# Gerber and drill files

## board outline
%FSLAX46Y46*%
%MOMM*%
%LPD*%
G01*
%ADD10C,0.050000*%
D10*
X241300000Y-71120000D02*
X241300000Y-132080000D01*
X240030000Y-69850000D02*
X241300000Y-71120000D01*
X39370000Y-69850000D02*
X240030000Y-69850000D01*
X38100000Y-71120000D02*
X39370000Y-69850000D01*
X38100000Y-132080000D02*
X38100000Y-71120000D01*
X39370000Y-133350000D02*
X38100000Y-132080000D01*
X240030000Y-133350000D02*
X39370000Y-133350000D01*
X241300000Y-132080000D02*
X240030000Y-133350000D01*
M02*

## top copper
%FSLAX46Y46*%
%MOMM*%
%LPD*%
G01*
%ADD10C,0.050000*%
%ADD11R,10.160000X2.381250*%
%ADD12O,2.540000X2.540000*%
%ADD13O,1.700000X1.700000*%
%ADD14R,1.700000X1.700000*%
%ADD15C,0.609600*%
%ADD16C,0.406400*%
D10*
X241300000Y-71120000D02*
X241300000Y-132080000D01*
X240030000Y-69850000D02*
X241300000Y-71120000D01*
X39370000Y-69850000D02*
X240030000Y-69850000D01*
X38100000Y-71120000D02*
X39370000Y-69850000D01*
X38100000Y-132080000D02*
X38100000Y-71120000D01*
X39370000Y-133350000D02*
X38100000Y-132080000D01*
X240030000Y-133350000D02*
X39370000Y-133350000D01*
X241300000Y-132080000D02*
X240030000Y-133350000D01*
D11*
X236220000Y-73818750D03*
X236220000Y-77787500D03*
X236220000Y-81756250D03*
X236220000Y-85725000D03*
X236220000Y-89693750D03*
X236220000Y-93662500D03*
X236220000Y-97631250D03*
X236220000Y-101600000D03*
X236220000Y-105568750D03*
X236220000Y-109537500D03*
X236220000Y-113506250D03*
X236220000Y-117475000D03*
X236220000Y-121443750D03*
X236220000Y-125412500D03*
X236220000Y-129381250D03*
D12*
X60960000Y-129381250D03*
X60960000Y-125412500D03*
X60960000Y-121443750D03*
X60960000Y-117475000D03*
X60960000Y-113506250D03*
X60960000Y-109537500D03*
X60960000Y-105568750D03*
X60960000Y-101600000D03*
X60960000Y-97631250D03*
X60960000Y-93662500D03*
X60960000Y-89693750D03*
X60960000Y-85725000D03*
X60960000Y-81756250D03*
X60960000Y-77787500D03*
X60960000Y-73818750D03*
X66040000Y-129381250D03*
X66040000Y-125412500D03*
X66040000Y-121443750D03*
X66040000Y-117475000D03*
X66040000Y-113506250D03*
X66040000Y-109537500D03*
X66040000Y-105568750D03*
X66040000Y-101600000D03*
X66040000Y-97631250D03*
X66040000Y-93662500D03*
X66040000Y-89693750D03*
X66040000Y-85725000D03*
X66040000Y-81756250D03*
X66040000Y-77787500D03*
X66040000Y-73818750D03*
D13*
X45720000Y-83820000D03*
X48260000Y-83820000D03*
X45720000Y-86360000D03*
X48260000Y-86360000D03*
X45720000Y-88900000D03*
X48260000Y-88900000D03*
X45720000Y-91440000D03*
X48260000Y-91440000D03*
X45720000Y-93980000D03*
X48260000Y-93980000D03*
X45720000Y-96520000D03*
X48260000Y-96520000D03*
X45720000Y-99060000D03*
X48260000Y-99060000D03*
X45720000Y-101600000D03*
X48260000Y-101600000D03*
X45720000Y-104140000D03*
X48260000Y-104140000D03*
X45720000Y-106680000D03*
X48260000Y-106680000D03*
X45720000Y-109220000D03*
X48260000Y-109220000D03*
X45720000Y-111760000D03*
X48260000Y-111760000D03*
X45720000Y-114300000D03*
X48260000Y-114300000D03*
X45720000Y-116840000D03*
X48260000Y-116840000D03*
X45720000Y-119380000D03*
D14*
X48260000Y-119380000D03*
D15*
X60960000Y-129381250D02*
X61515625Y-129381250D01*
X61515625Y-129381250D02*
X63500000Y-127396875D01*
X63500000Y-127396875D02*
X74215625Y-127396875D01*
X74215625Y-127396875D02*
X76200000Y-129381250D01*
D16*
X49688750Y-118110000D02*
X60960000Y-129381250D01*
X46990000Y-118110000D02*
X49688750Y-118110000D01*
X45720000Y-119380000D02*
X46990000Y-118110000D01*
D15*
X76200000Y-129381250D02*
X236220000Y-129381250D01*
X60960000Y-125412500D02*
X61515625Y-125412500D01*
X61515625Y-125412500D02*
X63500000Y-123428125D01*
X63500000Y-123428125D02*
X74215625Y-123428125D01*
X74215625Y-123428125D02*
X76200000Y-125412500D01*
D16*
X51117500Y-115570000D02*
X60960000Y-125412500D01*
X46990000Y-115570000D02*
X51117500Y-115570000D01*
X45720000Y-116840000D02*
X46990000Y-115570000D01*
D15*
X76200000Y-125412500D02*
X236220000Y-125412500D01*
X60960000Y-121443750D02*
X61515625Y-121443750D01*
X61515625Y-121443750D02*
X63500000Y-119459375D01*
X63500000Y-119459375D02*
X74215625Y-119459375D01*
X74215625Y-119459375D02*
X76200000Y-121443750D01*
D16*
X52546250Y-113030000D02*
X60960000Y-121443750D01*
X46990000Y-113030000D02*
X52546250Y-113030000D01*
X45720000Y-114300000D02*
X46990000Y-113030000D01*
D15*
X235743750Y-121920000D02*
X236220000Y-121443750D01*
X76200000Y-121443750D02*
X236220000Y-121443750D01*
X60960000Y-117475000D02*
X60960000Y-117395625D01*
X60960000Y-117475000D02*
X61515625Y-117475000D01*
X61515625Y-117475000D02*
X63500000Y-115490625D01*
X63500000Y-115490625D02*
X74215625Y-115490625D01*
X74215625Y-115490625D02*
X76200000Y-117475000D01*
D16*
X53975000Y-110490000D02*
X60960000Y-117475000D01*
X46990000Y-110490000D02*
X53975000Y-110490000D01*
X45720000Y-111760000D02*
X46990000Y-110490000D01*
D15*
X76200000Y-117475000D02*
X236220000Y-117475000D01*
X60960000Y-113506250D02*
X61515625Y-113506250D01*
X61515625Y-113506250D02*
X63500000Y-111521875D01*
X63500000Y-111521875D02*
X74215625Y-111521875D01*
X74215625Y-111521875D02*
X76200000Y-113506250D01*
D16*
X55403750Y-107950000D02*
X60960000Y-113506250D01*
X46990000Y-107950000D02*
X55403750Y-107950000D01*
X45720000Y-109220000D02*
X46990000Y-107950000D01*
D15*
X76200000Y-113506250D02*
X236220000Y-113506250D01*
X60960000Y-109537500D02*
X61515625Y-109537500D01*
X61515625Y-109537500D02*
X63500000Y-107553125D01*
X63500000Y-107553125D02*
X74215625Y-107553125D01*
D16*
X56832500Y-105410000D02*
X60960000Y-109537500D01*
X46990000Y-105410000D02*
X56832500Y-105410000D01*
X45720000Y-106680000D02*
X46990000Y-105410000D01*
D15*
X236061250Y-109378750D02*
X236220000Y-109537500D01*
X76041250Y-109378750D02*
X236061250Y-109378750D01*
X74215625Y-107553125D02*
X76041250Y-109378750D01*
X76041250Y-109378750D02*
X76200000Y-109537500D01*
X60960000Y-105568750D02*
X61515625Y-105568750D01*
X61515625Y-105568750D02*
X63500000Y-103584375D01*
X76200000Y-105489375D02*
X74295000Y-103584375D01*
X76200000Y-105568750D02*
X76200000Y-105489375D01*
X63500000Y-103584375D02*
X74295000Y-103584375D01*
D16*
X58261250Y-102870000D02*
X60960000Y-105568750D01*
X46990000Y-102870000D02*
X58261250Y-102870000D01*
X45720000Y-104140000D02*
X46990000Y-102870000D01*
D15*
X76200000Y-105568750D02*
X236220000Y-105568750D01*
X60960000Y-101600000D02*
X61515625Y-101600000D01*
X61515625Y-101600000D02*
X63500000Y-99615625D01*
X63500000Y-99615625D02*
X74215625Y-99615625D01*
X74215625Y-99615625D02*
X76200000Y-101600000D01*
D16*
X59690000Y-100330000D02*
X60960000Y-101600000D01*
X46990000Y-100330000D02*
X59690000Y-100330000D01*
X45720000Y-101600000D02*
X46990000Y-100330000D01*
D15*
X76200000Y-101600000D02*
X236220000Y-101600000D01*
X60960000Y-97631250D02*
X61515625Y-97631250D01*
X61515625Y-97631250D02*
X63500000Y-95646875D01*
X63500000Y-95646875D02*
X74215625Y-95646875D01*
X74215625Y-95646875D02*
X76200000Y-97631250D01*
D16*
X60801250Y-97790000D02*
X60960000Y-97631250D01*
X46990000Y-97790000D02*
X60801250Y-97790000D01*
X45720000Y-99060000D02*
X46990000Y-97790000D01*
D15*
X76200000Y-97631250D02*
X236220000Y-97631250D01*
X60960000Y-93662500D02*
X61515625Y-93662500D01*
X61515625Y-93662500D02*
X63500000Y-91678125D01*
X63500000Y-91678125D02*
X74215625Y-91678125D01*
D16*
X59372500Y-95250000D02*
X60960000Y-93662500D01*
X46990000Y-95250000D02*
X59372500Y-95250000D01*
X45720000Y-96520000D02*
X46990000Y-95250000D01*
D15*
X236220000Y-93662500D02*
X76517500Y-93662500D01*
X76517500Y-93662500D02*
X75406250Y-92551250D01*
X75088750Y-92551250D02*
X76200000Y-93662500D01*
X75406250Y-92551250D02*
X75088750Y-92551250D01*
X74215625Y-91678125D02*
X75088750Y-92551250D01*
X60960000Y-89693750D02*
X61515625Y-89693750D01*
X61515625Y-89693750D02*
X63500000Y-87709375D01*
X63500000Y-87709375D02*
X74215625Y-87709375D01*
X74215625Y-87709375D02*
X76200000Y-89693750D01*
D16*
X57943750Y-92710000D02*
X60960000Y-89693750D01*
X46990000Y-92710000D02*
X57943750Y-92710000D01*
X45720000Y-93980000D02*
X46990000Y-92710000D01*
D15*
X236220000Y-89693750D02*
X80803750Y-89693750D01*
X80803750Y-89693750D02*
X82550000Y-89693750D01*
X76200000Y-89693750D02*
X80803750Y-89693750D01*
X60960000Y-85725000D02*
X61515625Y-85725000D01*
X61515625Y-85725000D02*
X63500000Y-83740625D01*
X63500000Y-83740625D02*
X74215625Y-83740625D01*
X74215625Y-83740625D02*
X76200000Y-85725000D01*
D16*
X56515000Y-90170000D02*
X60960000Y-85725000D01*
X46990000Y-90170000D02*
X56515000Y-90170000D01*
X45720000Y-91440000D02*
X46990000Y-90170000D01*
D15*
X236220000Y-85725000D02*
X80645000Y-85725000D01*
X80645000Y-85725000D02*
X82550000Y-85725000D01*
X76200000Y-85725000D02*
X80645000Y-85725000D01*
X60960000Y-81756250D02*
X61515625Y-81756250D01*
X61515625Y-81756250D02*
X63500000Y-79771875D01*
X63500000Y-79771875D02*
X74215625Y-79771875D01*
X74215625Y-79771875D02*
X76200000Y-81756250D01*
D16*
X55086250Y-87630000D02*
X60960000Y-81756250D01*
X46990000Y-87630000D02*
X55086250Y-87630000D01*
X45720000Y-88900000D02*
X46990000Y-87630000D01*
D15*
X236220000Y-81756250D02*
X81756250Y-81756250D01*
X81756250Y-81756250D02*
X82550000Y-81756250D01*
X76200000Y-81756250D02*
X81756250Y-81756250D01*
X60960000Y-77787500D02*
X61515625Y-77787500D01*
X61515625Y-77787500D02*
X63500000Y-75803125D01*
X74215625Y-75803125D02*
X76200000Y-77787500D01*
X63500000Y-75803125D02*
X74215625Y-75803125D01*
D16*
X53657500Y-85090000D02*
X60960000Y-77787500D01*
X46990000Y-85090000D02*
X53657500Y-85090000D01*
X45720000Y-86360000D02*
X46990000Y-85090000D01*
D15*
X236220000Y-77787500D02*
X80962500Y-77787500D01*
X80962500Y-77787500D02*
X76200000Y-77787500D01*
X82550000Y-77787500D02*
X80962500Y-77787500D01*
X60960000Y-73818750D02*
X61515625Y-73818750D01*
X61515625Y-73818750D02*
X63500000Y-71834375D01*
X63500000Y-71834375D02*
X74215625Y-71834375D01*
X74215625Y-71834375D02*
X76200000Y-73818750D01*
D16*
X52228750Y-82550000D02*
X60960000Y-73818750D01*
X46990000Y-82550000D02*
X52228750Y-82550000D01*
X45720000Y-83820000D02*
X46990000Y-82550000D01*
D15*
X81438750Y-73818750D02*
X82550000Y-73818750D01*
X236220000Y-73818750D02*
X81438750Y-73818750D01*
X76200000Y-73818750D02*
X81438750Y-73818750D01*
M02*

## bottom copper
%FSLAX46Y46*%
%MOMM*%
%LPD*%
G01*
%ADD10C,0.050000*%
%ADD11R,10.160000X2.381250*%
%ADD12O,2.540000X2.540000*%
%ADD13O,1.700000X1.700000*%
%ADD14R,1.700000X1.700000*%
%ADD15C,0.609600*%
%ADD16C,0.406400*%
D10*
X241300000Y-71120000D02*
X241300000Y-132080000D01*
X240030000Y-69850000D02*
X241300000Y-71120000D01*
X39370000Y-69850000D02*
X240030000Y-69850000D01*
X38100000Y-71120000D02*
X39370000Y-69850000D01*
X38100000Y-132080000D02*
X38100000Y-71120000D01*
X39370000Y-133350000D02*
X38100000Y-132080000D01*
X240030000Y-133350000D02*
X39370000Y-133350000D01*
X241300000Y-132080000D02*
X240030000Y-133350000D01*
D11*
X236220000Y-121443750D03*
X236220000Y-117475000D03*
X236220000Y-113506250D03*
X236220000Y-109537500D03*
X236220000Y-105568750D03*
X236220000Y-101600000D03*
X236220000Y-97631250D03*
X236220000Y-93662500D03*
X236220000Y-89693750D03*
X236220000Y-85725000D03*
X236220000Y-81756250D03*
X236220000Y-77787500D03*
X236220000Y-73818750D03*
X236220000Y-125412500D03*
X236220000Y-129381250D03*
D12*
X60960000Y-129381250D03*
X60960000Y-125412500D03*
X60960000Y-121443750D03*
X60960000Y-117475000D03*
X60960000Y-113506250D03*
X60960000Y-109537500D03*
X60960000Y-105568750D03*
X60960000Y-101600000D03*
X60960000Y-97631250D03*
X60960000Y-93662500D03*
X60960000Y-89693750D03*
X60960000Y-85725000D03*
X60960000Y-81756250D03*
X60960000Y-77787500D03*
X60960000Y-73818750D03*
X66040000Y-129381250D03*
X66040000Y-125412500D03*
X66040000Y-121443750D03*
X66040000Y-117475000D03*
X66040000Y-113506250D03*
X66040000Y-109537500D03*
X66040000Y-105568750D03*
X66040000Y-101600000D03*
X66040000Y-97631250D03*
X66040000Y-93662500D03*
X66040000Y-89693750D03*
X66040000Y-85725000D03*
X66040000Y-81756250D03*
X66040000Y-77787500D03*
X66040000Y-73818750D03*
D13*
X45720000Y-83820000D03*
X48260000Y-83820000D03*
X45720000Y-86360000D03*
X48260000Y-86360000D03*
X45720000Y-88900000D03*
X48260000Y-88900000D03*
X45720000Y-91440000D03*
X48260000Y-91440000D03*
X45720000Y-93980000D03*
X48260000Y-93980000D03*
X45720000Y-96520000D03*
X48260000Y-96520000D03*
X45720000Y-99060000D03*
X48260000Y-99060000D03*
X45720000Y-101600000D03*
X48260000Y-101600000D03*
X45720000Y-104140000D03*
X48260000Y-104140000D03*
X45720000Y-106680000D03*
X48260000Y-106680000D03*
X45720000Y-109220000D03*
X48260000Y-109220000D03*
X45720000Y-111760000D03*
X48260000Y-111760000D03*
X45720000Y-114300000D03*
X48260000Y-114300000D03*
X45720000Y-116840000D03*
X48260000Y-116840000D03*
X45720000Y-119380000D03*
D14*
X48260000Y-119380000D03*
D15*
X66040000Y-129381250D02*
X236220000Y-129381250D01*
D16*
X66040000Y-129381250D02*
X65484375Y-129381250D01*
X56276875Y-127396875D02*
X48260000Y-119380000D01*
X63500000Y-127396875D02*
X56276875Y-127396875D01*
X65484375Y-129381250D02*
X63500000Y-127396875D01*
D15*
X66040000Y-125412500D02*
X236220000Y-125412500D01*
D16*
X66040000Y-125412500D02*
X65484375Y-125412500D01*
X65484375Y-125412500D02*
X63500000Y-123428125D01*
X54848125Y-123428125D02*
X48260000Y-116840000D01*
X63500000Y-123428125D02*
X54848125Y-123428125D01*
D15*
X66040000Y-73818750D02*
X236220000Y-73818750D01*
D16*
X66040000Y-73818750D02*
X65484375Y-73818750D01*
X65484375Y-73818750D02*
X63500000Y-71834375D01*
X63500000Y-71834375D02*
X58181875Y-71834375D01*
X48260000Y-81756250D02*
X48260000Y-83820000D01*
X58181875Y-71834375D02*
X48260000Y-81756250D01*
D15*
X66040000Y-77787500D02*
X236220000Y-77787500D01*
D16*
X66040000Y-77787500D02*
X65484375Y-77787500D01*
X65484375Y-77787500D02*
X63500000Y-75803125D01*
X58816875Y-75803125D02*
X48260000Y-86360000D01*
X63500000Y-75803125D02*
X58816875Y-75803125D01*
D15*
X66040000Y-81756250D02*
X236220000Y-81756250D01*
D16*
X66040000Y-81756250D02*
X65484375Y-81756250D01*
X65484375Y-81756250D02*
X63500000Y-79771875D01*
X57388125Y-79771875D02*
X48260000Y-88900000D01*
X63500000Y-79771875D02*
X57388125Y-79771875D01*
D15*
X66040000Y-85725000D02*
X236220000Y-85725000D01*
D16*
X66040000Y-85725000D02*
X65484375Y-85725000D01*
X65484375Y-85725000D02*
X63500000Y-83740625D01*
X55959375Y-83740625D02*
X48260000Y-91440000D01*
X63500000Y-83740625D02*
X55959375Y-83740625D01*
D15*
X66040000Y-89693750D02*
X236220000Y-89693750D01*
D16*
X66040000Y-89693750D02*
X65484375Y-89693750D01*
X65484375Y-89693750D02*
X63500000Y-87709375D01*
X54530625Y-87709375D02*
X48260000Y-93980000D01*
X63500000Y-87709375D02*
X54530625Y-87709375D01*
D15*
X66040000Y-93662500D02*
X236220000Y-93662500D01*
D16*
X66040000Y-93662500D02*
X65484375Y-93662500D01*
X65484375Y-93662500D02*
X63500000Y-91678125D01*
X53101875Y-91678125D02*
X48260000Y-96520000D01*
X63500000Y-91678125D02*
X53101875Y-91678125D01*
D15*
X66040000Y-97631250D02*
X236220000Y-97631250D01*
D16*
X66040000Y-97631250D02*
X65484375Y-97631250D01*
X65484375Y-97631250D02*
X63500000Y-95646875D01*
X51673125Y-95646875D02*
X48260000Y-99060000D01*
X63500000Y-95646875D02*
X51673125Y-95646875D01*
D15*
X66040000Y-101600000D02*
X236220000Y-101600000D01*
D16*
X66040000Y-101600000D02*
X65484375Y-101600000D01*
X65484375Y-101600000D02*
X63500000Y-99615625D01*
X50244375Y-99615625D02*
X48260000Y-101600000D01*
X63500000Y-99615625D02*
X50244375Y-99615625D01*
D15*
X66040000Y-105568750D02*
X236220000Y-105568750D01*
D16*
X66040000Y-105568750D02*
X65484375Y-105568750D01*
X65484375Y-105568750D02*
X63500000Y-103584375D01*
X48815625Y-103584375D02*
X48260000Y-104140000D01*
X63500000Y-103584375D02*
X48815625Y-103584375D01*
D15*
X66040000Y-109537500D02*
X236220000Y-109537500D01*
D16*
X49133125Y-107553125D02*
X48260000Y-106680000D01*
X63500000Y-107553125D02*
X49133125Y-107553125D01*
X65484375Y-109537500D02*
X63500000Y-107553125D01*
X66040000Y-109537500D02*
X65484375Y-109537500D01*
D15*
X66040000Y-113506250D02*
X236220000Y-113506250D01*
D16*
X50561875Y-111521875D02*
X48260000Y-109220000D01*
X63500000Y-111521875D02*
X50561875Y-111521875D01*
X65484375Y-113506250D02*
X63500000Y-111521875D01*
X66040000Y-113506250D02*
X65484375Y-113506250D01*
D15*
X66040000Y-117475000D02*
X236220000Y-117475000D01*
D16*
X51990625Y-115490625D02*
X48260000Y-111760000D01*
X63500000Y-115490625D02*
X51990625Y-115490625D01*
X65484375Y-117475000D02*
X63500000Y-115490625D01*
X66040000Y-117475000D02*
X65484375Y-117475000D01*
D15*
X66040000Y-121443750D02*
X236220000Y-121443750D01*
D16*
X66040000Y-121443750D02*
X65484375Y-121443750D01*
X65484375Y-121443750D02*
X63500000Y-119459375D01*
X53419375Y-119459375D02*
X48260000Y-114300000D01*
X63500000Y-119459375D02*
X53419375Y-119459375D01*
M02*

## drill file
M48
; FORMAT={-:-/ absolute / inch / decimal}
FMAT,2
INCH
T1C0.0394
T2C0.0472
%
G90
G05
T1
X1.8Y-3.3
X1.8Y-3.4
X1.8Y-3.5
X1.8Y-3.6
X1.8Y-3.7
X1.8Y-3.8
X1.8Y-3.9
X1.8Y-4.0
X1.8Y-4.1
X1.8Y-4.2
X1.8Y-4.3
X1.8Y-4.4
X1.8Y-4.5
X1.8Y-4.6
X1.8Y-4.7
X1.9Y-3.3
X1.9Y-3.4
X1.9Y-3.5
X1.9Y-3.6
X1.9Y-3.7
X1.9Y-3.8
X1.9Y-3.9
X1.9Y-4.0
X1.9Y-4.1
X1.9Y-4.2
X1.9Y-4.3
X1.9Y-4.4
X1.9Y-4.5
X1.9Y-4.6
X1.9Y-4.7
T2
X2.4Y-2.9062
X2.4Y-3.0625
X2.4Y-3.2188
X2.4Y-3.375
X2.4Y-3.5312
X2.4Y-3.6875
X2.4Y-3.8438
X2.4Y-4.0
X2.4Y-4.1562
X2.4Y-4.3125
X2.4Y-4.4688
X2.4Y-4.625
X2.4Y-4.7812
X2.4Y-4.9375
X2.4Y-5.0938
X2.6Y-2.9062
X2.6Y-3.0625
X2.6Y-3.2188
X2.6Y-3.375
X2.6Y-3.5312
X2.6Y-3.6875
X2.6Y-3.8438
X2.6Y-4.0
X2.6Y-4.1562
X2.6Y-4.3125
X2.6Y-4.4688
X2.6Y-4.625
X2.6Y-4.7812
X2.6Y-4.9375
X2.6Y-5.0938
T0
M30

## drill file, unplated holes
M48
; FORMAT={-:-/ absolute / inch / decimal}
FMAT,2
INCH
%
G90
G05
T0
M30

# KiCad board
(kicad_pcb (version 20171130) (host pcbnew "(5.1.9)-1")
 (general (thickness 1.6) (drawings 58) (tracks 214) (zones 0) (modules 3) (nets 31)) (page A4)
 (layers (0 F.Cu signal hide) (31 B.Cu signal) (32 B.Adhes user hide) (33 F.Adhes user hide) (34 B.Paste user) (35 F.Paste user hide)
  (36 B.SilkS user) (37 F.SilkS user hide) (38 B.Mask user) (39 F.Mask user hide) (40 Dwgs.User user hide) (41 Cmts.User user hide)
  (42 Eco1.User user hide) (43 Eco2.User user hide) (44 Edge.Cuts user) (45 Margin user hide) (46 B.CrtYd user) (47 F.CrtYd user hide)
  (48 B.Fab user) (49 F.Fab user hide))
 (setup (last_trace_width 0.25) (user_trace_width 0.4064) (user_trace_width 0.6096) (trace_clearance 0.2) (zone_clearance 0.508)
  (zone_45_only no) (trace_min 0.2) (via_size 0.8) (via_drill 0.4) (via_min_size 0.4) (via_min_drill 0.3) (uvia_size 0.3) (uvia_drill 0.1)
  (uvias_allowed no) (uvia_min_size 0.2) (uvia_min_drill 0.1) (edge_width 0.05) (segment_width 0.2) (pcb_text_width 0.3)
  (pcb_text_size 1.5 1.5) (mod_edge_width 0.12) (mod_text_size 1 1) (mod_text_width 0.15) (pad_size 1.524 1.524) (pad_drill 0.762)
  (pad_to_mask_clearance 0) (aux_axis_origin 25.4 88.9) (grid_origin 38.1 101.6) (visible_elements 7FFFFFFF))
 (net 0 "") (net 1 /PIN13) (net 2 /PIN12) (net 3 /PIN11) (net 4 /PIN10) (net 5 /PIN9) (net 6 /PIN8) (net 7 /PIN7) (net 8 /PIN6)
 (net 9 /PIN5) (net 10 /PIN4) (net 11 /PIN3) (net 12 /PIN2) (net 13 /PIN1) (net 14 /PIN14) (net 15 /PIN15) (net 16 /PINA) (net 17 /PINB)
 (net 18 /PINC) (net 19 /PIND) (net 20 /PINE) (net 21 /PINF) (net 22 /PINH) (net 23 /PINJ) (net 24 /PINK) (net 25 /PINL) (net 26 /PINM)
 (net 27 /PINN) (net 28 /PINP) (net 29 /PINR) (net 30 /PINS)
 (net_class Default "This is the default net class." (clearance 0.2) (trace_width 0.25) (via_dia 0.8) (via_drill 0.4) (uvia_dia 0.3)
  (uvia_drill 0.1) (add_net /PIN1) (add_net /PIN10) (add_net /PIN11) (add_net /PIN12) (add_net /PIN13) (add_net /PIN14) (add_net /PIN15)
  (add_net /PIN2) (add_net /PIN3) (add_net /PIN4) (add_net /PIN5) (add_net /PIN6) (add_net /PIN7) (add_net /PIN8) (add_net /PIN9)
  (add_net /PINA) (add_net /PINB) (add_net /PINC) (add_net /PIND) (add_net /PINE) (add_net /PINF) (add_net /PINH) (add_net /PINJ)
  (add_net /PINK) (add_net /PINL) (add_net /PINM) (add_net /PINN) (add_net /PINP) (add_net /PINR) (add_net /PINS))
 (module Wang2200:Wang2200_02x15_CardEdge (layer F.Cu) (at 241.3 101.6 90)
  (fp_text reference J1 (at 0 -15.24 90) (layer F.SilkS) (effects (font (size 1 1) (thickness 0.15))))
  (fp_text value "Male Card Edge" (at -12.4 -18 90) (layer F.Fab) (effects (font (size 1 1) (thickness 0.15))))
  (pad 13 connect rect (at -19.84375 -5.08 90) (size 2.38125 10.16) (layers B.Cu B.Mask) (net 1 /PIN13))
  (pad 12 connect rect (at -15.875 -5.08 90) (size 2.38125 10.16) (layers B.Cu B.Mask) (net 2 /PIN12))
  (pad 11 connect rect (at -11.90625 -5.08 90) (size 2.38125 10.16) (layers B.Cu B.Mask) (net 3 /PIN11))
  (pad 10 connect rect (at -7.9375 -5.08 90) (size 2.38125 10.16) (layers B.Cu B.Mask) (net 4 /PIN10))
  (pad 9 connect rect (at -3.96875 -5.08 90) (size 2.38125 10.16) (layers B.Cu B.Mask) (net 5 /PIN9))
  (pad 8 connect rect (at 0 -5.08 90) (size 2.38125 10.16) (layers B.Cu B.Mask) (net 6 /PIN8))
  (pad 7 connect rect (at 3.96875 -5.08 90) (size 2.38125 10.16) (layers B.Cu B.Mask) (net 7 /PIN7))
  (pad 6 connect rect (at 7.9375 -5.08 90) (size 2.38125 10.16) (layers B.Cu B.Mask) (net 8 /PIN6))
  (pad 5 connect rect (at 11.90625 -5.08 90) (size 2.38125 10.16) (layers B.Cu B.Mask) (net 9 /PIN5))
  (pad 4 connect rect (at 15.875 -5.08 90) (size 2.38125 10.16) (layers B.Cu B.Mask) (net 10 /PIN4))
  (pad 3 connect rect (at 19.84375 -5.08 90) (size 2.38125 10.16) (layers B.Cu B.Mask) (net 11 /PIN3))
  (pad 2 connect rect (at 23.8125 -5.08 90) (size 2.38125 10.16) (layers B.Cu B.Mask) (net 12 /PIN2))
  (pad 1 connect rect (at 27.78125 -5.08 90) (size 2.38125 10.16) (layers B.Cu B.Mask) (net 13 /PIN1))
  (pad 14 connect rect (at -23.8125 -5.08 90) (size 2.38125 10.16) (layers B.Cu B.Mask) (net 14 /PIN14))
  (pad 15 connect rect (at -27.78125 -5.08 90) (size 2.38125 10.16) (layers B.Cu B.Mask) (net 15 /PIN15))
  (pad A connect rect (at 27.78125 -5.08 90) (size 2.38125 10.16) (layers F.Cu F.Mask) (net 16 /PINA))
  (pad B connect rect (at 23.8125 -5.08 90) (size 2.38125 10.16) (layers F.Cu F.Mask) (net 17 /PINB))
  (pad C connect rect (at 19.84375 -5.08 90) (size 2.38125 10.16) (layers F.Cu F.Mask) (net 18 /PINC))
  (pad D connect rect (at 15.875 -5.08 90) (size 2.38125 10.16) (layers F.Cu F.Mask) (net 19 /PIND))
  (pad E connect rect (at 11.90625 -5.08 90) (size 2.38125 10.16) (layers F.Cu F.Mask) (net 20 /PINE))
  (pad F connect rect (at 7.9375 -5.08 90) (size 2.38125 10.16) (layers F.Cu F.Mask) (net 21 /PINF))
  (pad H connect rect (at 3.96875 -5.08 90) (size 2.38125 10.16) (layers F.Cu F.Mask) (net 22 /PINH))
  (pad J connect rect (at 0 -5.08 90) (size 2.38125 10.16) (layers F.Cu F.Mask) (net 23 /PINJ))
  (pad K connect rect (at -3.96875 -5.08 90) (size 2.38125 10.16) (layers F.Cu F.Mask) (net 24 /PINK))
  (pad L connect rect (at -7.9375 -5.08 90) (size 2.38125 10.16) (layers F.Cu F.Mask) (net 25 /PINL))
  (pad M connect rect (at -11.90625 -5.08 90) (size 2.38125 10.16) (layers F.Cu F.Mask) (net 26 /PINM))
  (pad N connect rect (at -15.875 -5.08 90) (size 2.38125 10.16) (layers F.Cu F.Mask) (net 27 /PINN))
  (pad P connect rect (at -19.84375 -5.08 90) (size 2.38125 10.16) (layers F.Cu F.Mask) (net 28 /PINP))
  (pad R connect rect (at -23.8125 -5.08 90) (size 2.38125 10.16) (layers F.Cu F.Mask) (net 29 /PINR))
  (pad S connect rect (at -27.78125 -5.08 90) (size 2.38125 10.16) (layers F.Cu F.Mask) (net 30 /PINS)))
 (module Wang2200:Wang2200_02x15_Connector (layer B.Cu) (at 63.5 101.6 90)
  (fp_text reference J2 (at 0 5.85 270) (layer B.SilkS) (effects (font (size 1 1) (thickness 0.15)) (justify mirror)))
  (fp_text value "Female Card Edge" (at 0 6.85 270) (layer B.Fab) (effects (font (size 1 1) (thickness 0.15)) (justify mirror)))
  (pad S thru_hole oval (at -27.78125 -2.54 90) (size 2.54 2.54) (drill 1.2) (layers *.Cu *.Mask) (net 30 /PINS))
  (pad R thru_hole oval (at -23.8125 -2.54 90) (size 2.54 2.54) (drill 1.2) (layers *.Cu *.Mask) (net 29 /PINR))
  (pad P thru_hole oval (at -19.84375 -2.54 90) (size 2.54 2.54) (drill 1.2) (layers *.Cu *.Mask) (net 28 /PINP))
  (pad N thru_hole oval (at -15.875 -2.54 90) (size 2.54 2.54) (drill 1.2) (layers *.Cu *.Mask) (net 27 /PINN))
  (pad M thru_hole oval (at -11.90625 -2.54 90) (size 2.54 2.54) (drill 1.2) (layers *.Cu *.Mask) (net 26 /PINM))
  (pad L thru_hole oval (at -7.9375 -2.54 90) (size 2.54 2.54) (drill 1.2) (layers *.Cu *.Mask) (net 25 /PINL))
  (pad K thru_hole oval (at -3.96875 -2.54 90) (size 2.54 2.54) (drill 1.2) (layers *.Cu *.Mask) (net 24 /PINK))
  (pad J thru_hole oval (at 0 -2.54 90) (size 2.54 2.54) (drill 1.2) (layers *.Cu *.Mask) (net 23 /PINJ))
  (pad H thru_hole oval (at 3.96875 -2.54 90) (size 2.54 2.54) (drill 1.2) (layers *.Cu *.Mask) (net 22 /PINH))
  (pad F thru_hole oval (at 7.9375 -2.54 90) (size 2.54 2.54) (drill 1.2) (layers *.Cu *.Mask) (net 21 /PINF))
  (pad E thru_hole oval (at 11.90625 -2.54 90) (size 2.54 2.54) (drill 1.2) (layers *.Cu *.Mask) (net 20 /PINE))
  (pad D thru_hole oval (at 15.875 -2.54 90) (size 2.54 2.54) (drill 1.2) (layers *.Cu *.Mask) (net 19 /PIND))
  (pad C thru_hole oval (at 19.84375 -2.54 90) (size 2.54 2.54) (drill 1.2) (layers *.Cu *.Mask) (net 18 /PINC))
  (pad B thru_hole oval (at 23.8125 -2.54 90) (size 2.54 2.54) (drill 1.2) (layers *.Cu *.Mask) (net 17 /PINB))
  (pad A thru_hole oval (at 27.78125 -2.54 90) (size 2.54 2.54) (drill 1.2) (layers *.Cu *.Mask) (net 16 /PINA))
  (pad 15 thru_hole oval (at -27.78125 2.54 90) (size 2.54 2.54) (drill 1.2) (layers *.Cu *.Mask) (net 15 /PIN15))
  (pad 14 thru_hole oval (at -23.8125 2.54 90) (size 2.54 2.54) (drill 1.2) (layers *.Cu *.Mask) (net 14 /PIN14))
  (pad 13 thru_hole oval (at -19.84375 2.54 90) (size 2.54 2.54) (drill 1.2) (layers *.Cu *.Mask) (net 1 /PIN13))
  (pad 12 thru_hole oval (at -15.875 2.54 90) (size 2.54 2.54) (drill 1.2) (layers *.Cu *.Mask) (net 2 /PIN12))
  (pad 11 thru_hole oval (at -11.90625 2.54 90) (size 2.54 2.54) (drill 1.2) (layers *.Cu *.Mask) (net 3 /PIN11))
  (pad 10 thru_hole oval (at -7.9375 2.54 90) (size 2.54 2.54) (drill 1.2) (layers *.Cu *.Mask) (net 4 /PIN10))
  (pad 9 thru_hole oval (at -3.96875 2.54 90) (size 2.54 2.54) (drill 1.2) (layers *.Cu *.Mask) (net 5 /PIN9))
  (pad 8 thru_hole oval (at 0 2.54 90) (size 2.54 2.54) (drill 1.2) (layers *.Cu *.Mask) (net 6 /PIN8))
  (pad 7 thru_hole oval (at 3.96875 2.54 90) (size 2.54 2.54) (drill 1.2) (layers *.Cu *.Mask) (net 7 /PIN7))
  (pad 6 thru_hole oval (at 7.9375 2.54 90) (size 2.54 2.54) (drill 1.2) (layers *.Cu *.Mask) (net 8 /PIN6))
  (pad 5 thru_hole oval (at 11.90625 2.54 90) (size 2.54 2.54) (drill 1.2) (layers *.Cu *.Mask) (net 9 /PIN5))
  (pad 4 thru_hole oval (at 15.875 2.54 90) (size 2.54 2.54) (drill 1.2) (layers *.Cu *.Mask) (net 10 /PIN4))
  (pad 3 thru_hole oval (at 19.84375 2.54 90) (size 2.54 2.54) (drill 1.2) (layers *.Cu *.Mask) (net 11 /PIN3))
  (pad 2 thru_hole oval (at 23.8125 2.54 90) (size 2.54 2.54) (drill 1.2) (layers *.Cu *.Mask) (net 12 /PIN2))
  (pad 1 thru_hole oval (at 27.78125 2.54 90) (size 2.54 2.54) (drill 1.2) (layers *.Cu *.Mask) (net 13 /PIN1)))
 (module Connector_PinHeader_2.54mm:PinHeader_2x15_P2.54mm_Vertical (layer F.Cu) (at 48.26 119.38 180)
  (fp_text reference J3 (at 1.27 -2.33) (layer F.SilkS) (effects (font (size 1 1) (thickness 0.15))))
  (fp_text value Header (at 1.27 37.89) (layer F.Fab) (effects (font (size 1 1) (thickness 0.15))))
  (pad 30 thru_hole oval (at 2.54 35.56 180) (size 1.7 1.7) (drill 1) (layers *.Cu *.Mask) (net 16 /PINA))
  (pad 29 thru_hole oval (at 0 35.56 180) (size 1.7 1.7) (drill 1) (layers *.Cu *.Mask) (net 13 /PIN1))
  (pad 28 thru_hole oval (at 2.54 33.02 180) (size 1.7 1.7) (drill 1) (layers *.Cu *.Mask) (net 17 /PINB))
  (pad 27 thru_hole oval (at 0 33.02 180) (size 1.7 1.7) (drill 1) (layers *.Cu *.Mask) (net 12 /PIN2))
  (pad 26 thru_hole oval (at 2.54 30.48 180) (size 1.7 1.7) (drill 1) (layers *.Cu *.Mask) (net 18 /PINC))
  (pad 25 thru_hole oval (at 0 30.48 180) (size 1.7 1.7) (drill 1) (layers *.Cu *.Mask) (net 11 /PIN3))
  (pad 24 thru_hole oval (at 2.54 27.94 180) (size 1.7 1.7) (drill 1) (layers *.Cu *.Mask) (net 19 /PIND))
  (pad 23 thru_hole oval (at 0 27.94 180) (size 1.7 1.7) (drill 1) (layers *.Cu *.Mask) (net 10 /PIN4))
  (pad 22 thru_hole oval (at 2.54 25.4 180) (size 1.7 1.7) (drill 1) (layers *.Cu *.Mask) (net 20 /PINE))
  (pad 21 thru_hole oval (at 0 25.4 180) (size 1.7 1.7) (drill 1) (layers *.Cu *.Mask) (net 9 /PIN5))
  (pad 20 thru_hole oval (at 2.54 22.86 180) (size 1.7 1.7) (drill 1) (layers *.Cu *.Mask) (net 21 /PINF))
  (pad 19 thru_hole oval (at 0 22.86 180) (size 1.7 1.7) (drill 1) (layers *.Cu *.Mask) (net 8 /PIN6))
  (pad 18 thru_hole oval (at 2.54 20.32 180) (size 1.7 1.7) (drill 1) (layers *.Cu *.Mask) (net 22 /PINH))
  (pad 17 thru_hole oval (at 0 20.32 180) (size 1.7 1.7) (drill 1) (layers *.Cu *.Mask) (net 7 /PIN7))
  (pad 16 thru_hole oval (at 2.54 17.78 180) (size 1.7 1.7) (drill 1) (layers *.Cu *.Mask) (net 23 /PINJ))
  (pad 15 thru_hole oval (at 0 17.78 180) (size 1.7 1.7) (drill 1) (layers *.Cu *.Mask) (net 6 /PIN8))
  (pad 14 thru_hole oval (at 2.54 15.24 180) (size 1.7 1.7) (drill 1) (layers *.Cu *.Mask) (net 24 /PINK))
  (pad 13 thru_hole oval (at 0 15.24 180) (size 1.7 1.7) (drill 1) (layers *.Cu *.Mask) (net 5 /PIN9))
  (pad 12 thru_hole oval (at 2.54 12.7 180) (size 1.7 1.7) (drill 1) (layers *.Cu *.Mask) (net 25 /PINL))
  (pad 11 thru_hole oval (at 0 12.7 180) (size 1.7 1.7) (drill 1) (layers *.Cu *.Mask) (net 4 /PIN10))
  (pad 10 thru_hole oval (at 2.54 10.16 180) (size 1.7 1.7) (drill 1) (layers *.Cu *.Mask) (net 26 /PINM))
  (pad 9 thru_hole oval (at 0 10.16 180) (size 1.7 1.7) (drill 1) (layers *.Cu *.Mask) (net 3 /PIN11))
  (pad 8 thru_hole oval (at 2.54 7.62 180) (size 1.7 1.7) (drill 1) (layers *.Cu *.Mask) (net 27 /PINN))
  (pad 7 thru_hole oval (at 0 7.62 180) (size 1.7 1.7) (drill 1) (layers *.Cu *.Mask) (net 2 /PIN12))
  (pad 6 thru_hole oval (at 2.54 5.08 180) (size 1.7 1.7) (drill 1) (layers *.Cu *.Mask) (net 28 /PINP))
  (pad 5 thru_hole oval (at 0 5.08 180) (size 1.7 1.7) (drill 1) (layers *.Cu *.Mask) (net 1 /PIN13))
  (pad 4 thru_hole oval (at 2.54 2.54 180) (size 1.7 1.7) (drill 1) (layers *.Cu *.Mask) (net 29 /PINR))
  (pad 3 thru_hole oval (at 0 2.54 180) (size 1.7 1.7) (drill 1) (layers *.Cu *.Mask) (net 14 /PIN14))
  (pad 2 thru_hole oval (at 2.54 0 180) (size 1.7 1.7) (drill 1) (layers *.Cu *.Mask) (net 30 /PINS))
  (pad 1 thru_hole rect (at 0 0 180) (size 1.7 1.7) (drill 1) (layers *.Cu *.Mask) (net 15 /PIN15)))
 (gr_line (start 241.3 71.12) (end 241.3 132.08) (layer Edge.Cuts) (width 0.05))
 (gr_line (start 240.03 69.85) (end 241.3 71.12) (layer Edge.Cuts) (width 0.05))
 (gr_line (start 39.37 69.85) (end 240.03 69.85) (layer Edge.Cuts) (width 0.05))
 (gr_line (start 38.1 71.12) (end 39.37 69.85) (layer Edge.Cuts) (width 0.05))
 (gr_line (start 38.1 132.08) (end 38.1 71.12) (layer Edge.Cuts) (width 0.05))
 (gr_line (start 39.37 133.35) (end 38.1 132.08) (layer Edge.Cuts) (width 0.05))
 (gr_line (start 240.03 133.35) (end 39.37 133.35) (layer Edge.Cuts) (width 0.05))
 (gr_line (start 241.3 132.08) (end 240.03 133.35) (layer Edge.Cuts) (width 0.05))
 (segment (start 60.96 129.38125) (end 61.515625 129.38125) (width 0.6096) (layer F.Cu) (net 30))
 (segment (start 61.515625 129.38125) (end 63.5 127.396875) (width 0.6096) (layer F.Cu) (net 30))
 (segment (start 63.5 127.396875) (end 74.215625 127.396875) (width 0.6096) (layer F.Cu) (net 30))
 (segment (start 74.215625 127.396875) (end 76.2 129.38125) (width 0.6096) (layer F.Cu) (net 30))
 (segment (start 49.68875 118.11) (end 60.96 129.38125) (width 0.4064) (layer F.Cu) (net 30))
 (segment (start 46.99 118.11) (end 49.68875 118.11) (width 0.4064) (layer F.Cu) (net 30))
 (segment (start 45.72 119.38) (end 46.99 118.11) (width 0.4064) (layer F.Cu) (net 30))
 (segment (start 76.2 129.38125) (end 236.22 129.38125) (width 0.6096) (layer F.Cu) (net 30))
 (segment (start 60.96 125.4125) (end 61.515625 125.4125) (width 0.6096) (layer F.Cu) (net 29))
 (segment (start 61.515625 125.4125) (end 63.5 123.428125) (width 0.6096) (layer F.Cu) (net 29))
 (segment (start 63.5 123.428125) (end 74.215625 123.428125) (width 0.6096) (layer F.Cu) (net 29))
 (segment (start 74.215625 123.428125) (end 76.2 125.4125) (width 0.6096) (layer F.Cu) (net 29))
 (segment (start 51.1175 115.57) (end 60.96 125.4125) (width 0.4064) (layer F.Cu) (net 29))
 (segment (start 46.99 115.57) (end 51.1175 115.57) (width 0.4064) (layer F.Cu) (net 29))
 (segment (start 45.72 116.84) (end 46.99 115.57) (width 0.4064) (layer F.Cu) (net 29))
 (segment (start 76.2 125.4125) (end 236.22 125.4125) (width 0.6096) (layer F.Cu) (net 29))
 (segment (start 60.96 121.44375) (end 61.515625 121.44375) (width 0.6096) (layer F.Cu) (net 28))
 (segment (start 61.515625 121.44375) (end 63.5 119.459375) (width 0.6096) (layer F.Cu) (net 28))
 (segment (start 63.5 119.459375) (end 74.215625 119.459375) (width 0.6096) (layer F.Cu) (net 28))
 (segment (start 74.215625 119.459375) (end 76.2 121.44375) (width 0.6096) (layer F.Cu) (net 28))
 (segment (start 52.54625 113.03) (end 60.96 121.44375) (width 0.4064) (layer F.Cu) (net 28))
 (segment (start 46.99 113.03) (end 52.54625 113.03) (width 0.4064) (layer F.Cu) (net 28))
 (segment (start 45.72 114.3) (end 46.99 113.03) (width 0.4064) (layer F.Cu) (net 28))
 (segment (start 235.74375 121.92) (end 236.22 121.44375) (width 0.6096) (layer F.Cu) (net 28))
 (segment (start 76.2 121.44375) (end 236.22 121.44375) (width 0.6096) (layer F.Cu) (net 28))
 (segment (start 60.96 117.475) (end 60.96 117.395625) (width 0.6096) (layer F.Cu) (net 27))
 (segment (start 60.96 117.475) (end 61.515625 117.475) (width 0.6096) (layer F.Cu) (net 27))
 (segment (start 61.515625 117.475) (end 63.5 115.490625) (width 0.6096) (layer F.Cu) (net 27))
 (segment (start 63.5 115.490625) (end 74.215625 115.490625) (width 0.6096) (layer F.Cu) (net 27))
 (segment (start 74.215625 115.490625) (end 76.2 117.475) (width 0.6096) (layer F.Cu) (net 27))
 (segment (start 53.975 110.49) (end 60.96 117.475) (width 0.4064) (layer F.Cu) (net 27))
 (segment (start 46.99 110.49) (end 53.975 110.49) (width 0.4064) (layer F.Cu) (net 27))
 (segment (start 45.72 111.76) (end 46.99 110.49) (width 0.4064) (layer F.Cu) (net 27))
 (segment (start 76.2 117.475) (end 236.22 117.475) (width 0.6096) (layer F.Cu) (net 27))
 (segment (start 60.96 113.50625) (end 61.515625 113.50625) (width 0.6096) (layer F.Cu) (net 26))
 (segment (start 61.515625 113.50625) (end 63.5 111.521875) (width 0.6096) (layer F.Cu) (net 26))
 (segment (start 63.5 111.521875) (end 74.215625 111.521875) (width 0.6096) (layer F.Cu) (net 26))
 (segment (start 74.215625 111.521875) (end 76.2 113.50625) (width 0.6096) (layer F.Cu) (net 26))
 (segment (start 55.40375 107.95) (end 60.96 113.50625) (width 0.4064) (layer F.Cu) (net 26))
 (segment (start 46.99 107.95) (end 55.40375 107.95) (width 0.4064) (layer F.Cu) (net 26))
 (segment (start 45.72 109.22) (end 46.99 107.95) (width 0.4064) (layer F.Cu) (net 26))
 (segment (start 76.2 113.50625) (end 236.22 113.50625) (width 0.6096) (layer F.Cu) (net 26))
 (segment (start 60.96 109.5375) (end 61.515625 109.5375) (width 0.6096) (layer F.Cu) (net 25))
 (segment (start 61.515625 109.5375) (end 63.5 107.553125) (width 0.6096) (layer F.Cu) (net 25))
 (segment (start 63.5 107.553125) (end 74.215625 107.553125) (width 0.6096) (layer F.Cu) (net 25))
 (segment (start 56.8325 105.41) (end 60.96 109.5375) (width 0.4064) (layer F.Cu) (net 25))
 (segment (start 46.99 105.41) (end 56.8325 105.41) (width 0.4064) (layer F.Cu) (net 25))
 (segment (start 45.72 106.68) (end 46.99 105.41) (width 0.4064) (layer F.Cu) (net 25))
 (segment (start 236.06125 109.37875) (end 236.22 109.5375) (width 0.6096) (layer F.Cu) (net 25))
 (segment (start 76.04125 109.37875) (end 236.06125 109.37875) (width 0.6096) (layer F.Cu) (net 25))
 (segment (start 74.215625 107.553125) (end 76.04125 109.37875) (width 0.6096) (layer F.Cu) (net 25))
 (segment (start 76.04125 109.37875) (end 76.2 109.5375) (width 0.6096) (layer F.Cu) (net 25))
 (segment (start 60.96 105.56875) (end 61.515625 105.56875) (width 0.6096) (layer F.Cu) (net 24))
 (segment (start 61.515625 105.56875) (end 63.5 103.584375) (width 0.6096) (layer F.Cu) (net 24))
 (segment (start 76.2 105.489375) (end 74.295 103.584375) (width 0.6096) (layer F.Cu) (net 24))
 (segment (start 76.2 105.56875) (end 76.2 105.489375) (width 0.6096) (layer F.Cu) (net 24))
 (segment (start 63.5 103.584375) (end 74.295 103.584375) (width 0.6096) (layer F.Cu) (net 24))
 (segment (start 58.26125 102.87) (end 60.96 105.56875) (width 0.4064) (layer F.Cu) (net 24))
 (segment (start 46.99 102.87) (end 58.26125 102.87) (width 0.4064) (layer F.Cu) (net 24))
 (segment (start 45.72 104.14) (end 46.99 102.87) (width 0.4064) (layer F.Cu) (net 24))
 (segment (start 76.2 105.56875) (end 236.22 105.56875) (width 0.6096) (layer F.Cu) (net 24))
 (segment (start 60.96 101.6) (end 61.515625 101.6) (width 0.6096) (layer F.Cu) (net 23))
 (segment (start 61.515625 101.6) (end 63.5 99.615625) (width 0.6096) (layer F.Cu) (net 23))
 (segment (start 63.5 99.615625) (end 74.215625 99.615625) (width 0.6096) (layer F.Cu) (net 23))
 (segment (start 74.215625 99.615625) (end 76.2 101.6) (width 0.6096) (layer F.Cu) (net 23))
 (segment (start 59.69 100.33) (end 60.96 101.6) (width 0.4064) (layer F.Cu) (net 23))
 (segment (start 46.99 100.33) (end 59.69 100.33) (width 0.4064) (layer F.Cu) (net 23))
 (segment (start 45.72 101.6) (end 46.99 100.33) (width 0.4064) (layer F.Cu) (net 23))
 (segment (start 76.2 101.6) (end 236.22 101.6) (width 0.6096) (layer F.Cu) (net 23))
 (segment (start 60.96 97.63125) (end 61.515625 97.63125) (width 0.6096) (layer F.Cu) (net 22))
 (segment (start 61.515625 97.63125) (end 63.5 95.646875) (width 0.6096) (layer F.Cu) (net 22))
 (segment (start 63.5 95.646875) (end 74.215625 95.646875) (width 0.6096) (layer F.Cu) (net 22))
 (segment (start 74.215625 95.646875) (end 76.2 97.63125) (width 0.6096) (layer F.Cu) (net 22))
 (segment (start 60.80125 97.79) (end 60.96 97.63125) (width 0.4064) (layer F.Cu) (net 22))
 (segment (start 46.99 97.79) (end 60.80125 97.79) (width 0.4064) (layer F.Cu) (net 22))
 (segment (start 45.72 99.06) (end 46.99 97.79) (width 0.4064) (layer F.Cu) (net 22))
 (segment (start 76.2 97.63125) (end 236.22 97.63125) (width 0.6096) (layer F.Cu) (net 22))
 (segment (start 60.96 93.6625) (end 61.515625 93.6625) (width 0.6096) (layer F.Cu) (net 21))
 (segment (start 61.515625 93.6625) (end 63.5 91.678125) (width 0.6096) (layer F.Cu) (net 21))
 (segment (start 63.5 91.678125) (end 74.215625 91.678125) (width 0.6096) (layer F.Cu) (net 21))
 (segment (start 59.3725 95.25) (end 60.96 93.6625) (width 0.4064) (layer F.Cu) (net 21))
 (segment (start 46.99 95.25) (end 59.3725 95.25) (width 0.4064) (layer F.Cu) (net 21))
 (segment (start 45.72 96.52) (end 46.99 95.25) (width 0.4064) (layer F.Cu) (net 21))
 (segment (start 236.22 93.6625) (end 76.5175 93.6625) (width 0.6096) (layer F.Cu) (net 21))
 (segment (start 76.5175 93.6625) (end 75.40625 92.55125) (width 0.6096) (layer F.Cu) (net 21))
 (segment (start 75.08875 92.55125) (end 76.2 93.6625) (width 0.6096) (layer F.Cu) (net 21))
 (segment (start 75.40625 92.55125) (end 75.08875 92.55125) (width 0.6096) (layer F.Cu) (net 21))
 (segment (start 74.215625 91.678125) (end 75.08875 92.55125) (width 0.6096) (layer F.Cu) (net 21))
 (segment (start 60.96 89.69375) (end 61.515625 89.69375) (width 0.6096) (layer F.Cu) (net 20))
 (segment (start 61.515625 89.69375) (end 63.5 87.709375) (width 0.6096) (layer F.Cu) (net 20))
 (segment (start 63.5 87.709375) (end 74.215625 87.709375) (width 0.6096) (layer F.Cu) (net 20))
 (segment (start 74.215625 87.709375) (end 76.2 89.69375) (width 0.6096) (layer F.Cu) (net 20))
 (segment (start 57.94375 92.71) (end 60.96 89.69375) (width 0.4064) (layer F.Cu) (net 20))
 (segment (start 46.99 92.71) (end 57.94375 92.71) (width 0.4064) (layer F.Cu) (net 20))
 (segment (start 45.72 93.98) (end 46.99 92.71) (width 0.4064) (layer F.Cu) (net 20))
 (segment (start 236.22 89.69375) (end 80.80375 89.69375) (width 0.6096) (layer F.Cu) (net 20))
 (segment (start 80.80375 89.69375) (end 82.55 89.69375) (width 0.6096) (layer F.Cu) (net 20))
 (segment (start 76.2 89.69375) (end 80.80375 89.69375) (width 0.6096) (layer F.Cu) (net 20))
 (segment (start 60.96 85.725) (end 61.515625 85.725) (width 0.6096) (layer F.Cu) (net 19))
 (segment (start 61.515625 85.725) (end 63.5 83.740625) (width 0.6096) (layer F.Cu) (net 19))
 (segment (start 63.5 83.740625) (end 74.215625 83.740625) (width 0.6096) (layer F.Cu) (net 19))
 (segment (start 74.215625 83.740625) (end 76.2 85.725) (width 0.6096) (layer F.Cu) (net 19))
 (segment (start 56.515 90.17) (end 60.96 85.725) (width 0.4064) (layer F.Cu) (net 19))
 (segment (start 46.99 90.17) (end 56.515 90.17) (width 0.4064) (layer F.Cu) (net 19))
 (segment (start 45.72 91.44) (end 46.99 90.17) (width 0.4064) (layer F.Cu) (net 19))
 (segment (start 236.22 85.725) (end 80.645 85.725) (width 0.6096) (layer F.Cu) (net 19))
 (segment (start 80.645 85.725) (end 82.55 85.725) (width 0.6096) (layer F.Cu) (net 19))
 (segment (start 76.2 85.725) (end 80.645 85.725) (width 0.6096) (layer F.Cu) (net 19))
 (segment (start 60.96 81.75625) (end 61.515625 81.75625) (width 0.6096) (layer F.Cu) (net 18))
 (segment (start 61.515625 81.75625) (end 63.5 79.771875) (width 0.6096) (layer F.Cu) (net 18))
 (segment (start 63.5 79.771875) (end 74.215625 79.771875) (width 0.6096) (layer F.Cu) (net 18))
 (segment (start 74.215625 79.771875) (end 76.2 81.75625) (width 0.6096) (layer F.Cu) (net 18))
 (segment (start 55.08625 87.63) (end 60.96 81.75625) (width 0.4064) (layer F.Cu) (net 18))
 (segment (start 46.99 87.63) (end 55.08625 87.63) (width 0.4064) (layer F.Cu) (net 18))
 (segment (start 45.72 88.9) (end 46.99 87.63) (width 0.4064) (layer F.Cu) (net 18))
 (segment (start 236.22 81.75625) (end 81.75625 81.75625) (width 0.6096) (layer F.Cu) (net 18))
 (segment (start 81.75625 81.75625) (end 82.55 81.75625) (width 0.6096) (layer F.Cu) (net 18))
 (segment (start 76.2 81.75625) (end 81.75625 81.75625) (width 0.6096) (layer F.Cu) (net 18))
 (segment (start 60.96 77.7875) (end 61.515625 77.7875) (width 0.6096) (layer F.Cu) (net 17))
 (segment (start 61.515625 77.7875) (end 63.5 75.803125) (width 0.6096) (layer F.Cu) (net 17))
 (segment (start 74.215625 75.803125) (end 76.2 77.7875) (width 0.6096) (layer F.Cu) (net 17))
 (segment (start 63.5 75.803125) (end 74.215625 75.803125) (width 0.6096) (layer F.Cu) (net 17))
 (segment (start 53.6575 85.09) (end 60.96 77.7875) (width 0.4064) (layer F.Cu) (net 17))
 (segment (start 46.99 85.09) (end 53.6575 85.09) (width 0.4064) (layer F.Cu) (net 17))
 (segment (start 45.72 86.36) (end 46.99 85.09) (width 0.4064) (layer F.Cu) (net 17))
 (segment (start 236.22 77.7875) (end 80.9625 77.7875) (width 0.6096) (layer F.Cu) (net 17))
 (segment (start 80.9625 77.7875) (end 76.2 77.7875) (width 0.6096) (layer F.Cu) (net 17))
 (segment (start 82.55 77.7875) (end 80.9625 77.7875) (width 0.6096) (layer F.Cu) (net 17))
 (segment (start 60.96 73.81875) (end 61.515625 73.81875) (width 0.6096) (layer F.Cu) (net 16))
 (segment (start 61.515625 73.81875) (end 63.5 71.834375) (width 0.6096) (layer F.Cu) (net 16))
 (segment (start 63.5 71.834375) (end 74.215625 71.834375) (width 0.6096) (layer F.Cu) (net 16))
 (segment (start 74.215625 71.834375) (end 76.2 73.81875) (width 0.6096) (layer F.Cu) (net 16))
 (segment (start 52.22875 82.55) (end 60.96 73.81875) (width 0.4064) (layer F.Cu) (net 16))
 (segment (start 46.99 82.55) (end 52.22875 82.55) (width 0.4064) (layer F.Cu) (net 16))
 (segment (start 45.72 83.82) (end 46.99 82.55) (width 0.4064) (layer F.Cu) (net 16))
 (segment (start 81.43875 73.81875) (end 82.55 73.81875) (width 0.6096) (layer F.Cu) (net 16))
 (segment (start 236.22 73.81875) (end 81.43875 73.81875) (width 0.6096) (layer F.Cu) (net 16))
 (segment (start 76.2 73.81875) (end 81.43875 73.81875) (width 0.6096) (layer F.Cu) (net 16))
 (segment (start 66.04 129.38125) (end 236.22 129.38125) (width 0.6096) (layer B.Cu) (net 15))
 (segment (start 66.04 129.38125) (end 65.484375 129.38125) (width 0.4064) (layer B.Cu) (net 15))
 (segment (start 56.276875 127.396875) (end 48.26 119.38) (width 0.4064) (layer B.Cu) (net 15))
 (segment (start 63.5 127.396875) (end 56.276875 127.396875) (width 0.4064) (layer B.Cu) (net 15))
 (segment (start 65.484375 129.38125) (end 63.5 127.396875) (width 0.4064) (layer B.Cu) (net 15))
 (segment (start 66.04 125.4125) (end 236.22 125.4125) (width 0.6096) (layer B.Cu) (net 14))
 (segment (start 66.04 125.4125) (end 65.484375 125.4125) (width 0.4064) (layer B.Cu) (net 14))
 (segment (start 65.484375 125.4125) (end 63.5 123.428125) (width 0.4064) (layer B.Cu) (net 14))
 (segment (start 54.848125 123.428125) (end 48.26 116.84) (width 0.4064) (layer B.Cu) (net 14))
 (segment (start 63.5 123.428125) (end 54.848125 123.428125) (width 0.4064) (layer B.Cu) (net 14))
 (segment (start 66.04 73.81875) (end 236.22 73.81875) (width 0.6096) (layer B.Cu) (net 13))
 (segment (start 66.04 73.81875) (end 65.484375 73.81875) (width 0.4064) (layer B.Cu) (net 13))
 (segment (start 65.484375 73.81875) (end 63.5 71.834375) (width 0.4064) (layer B.Cu) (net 13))
 (segment (start 63.5 71.834375) (end 58.181875 71.834375) (width 0.4064) (layer B.Cu) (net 13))
 (segment (start 48.26 81.75625) (end 48.26 83.82) (width 0.4064) (layer B.Cu) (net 13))
 (segment (start 58.181875 71.834375) (end 48.26 81.75625) (width 0.4064) (layer B.Cu) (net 13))
 (segment (start 66.04 77.7875) (end 236.22 77.7875) (width 0.6096) (layer B.Cu) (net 12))
 (segment (start 66.04 77.7875) (end 65.484375 77.7875) (width 0.4064) (layer B.Cu) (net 12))
 (segment (start 65.484375 77.7875) (end 63.5 75.803125) (width 0.4064) (layer B.Cu) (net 12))
 (segment (start 58.816875 75.803125) (end 48.26 86.36) (width 0.4064) (layer B.Cu) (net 12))
 (segment (start 63.5 75.803125) (end 58.816875 75.803125) (width 0.4064) (layer B.Cu) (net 12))
 (segment (start 66.04 81.75625) (end 236.22 81.75625) (width 0.6096) (layer B.Cu) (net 11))
 (segment (start 66.04 81.75625) (end 65.484375 81.75625) (width 0.4064) (layer B.Cu) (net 11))
 (segment (start 65.484375 81.75625) (end 63.5 79.771875) (width 0.4064) (layer B.Cu) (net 11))
 (segment (start 57.388125 79.771875) (end 48.26 88.9) (width 0.4064) (layer B.Cu) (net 11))
 (segment (start 63.5 79.771875) (end 57.388125 79.771875) (width 0.4064) (layer B.Cu) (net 11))
 (segment (start 66.04 85.725) (end 236.22 85.725) (width 0.6096) (layer B.Cu) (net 10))
 (segment (start 66.04 85.725) (end 65.484375 85.725) (width 0.4064) (layer B.Cu) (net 10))
 (segment (start 65.484375 85.725) (end 63.5 83.740625) (width 0.4064) (layer B.Cu) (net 10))
 (segment (start 55.959375 83.740625) (end 48.26 91.44) (width 0.4064) (layer B.Cu) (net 10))
 (segment (start 63.5 83.740625) (end 55.959375 83.740625) (width 0.4064) (layer B.Cu) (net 10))
 (segment (start 66.04 89.69375) (end 236.22 89.69375) (width 0.6096) (layer B.Cu) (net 9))
 (segment (start 66.04 89.69375) (end 65.484375 89.69375) (width 0.4064) (layer B.Cu) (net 9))
 (segment (start 65.484375 89.69375) (end 63.5 87.709375) (width 0.4064) (layer B.Cu) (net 9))
 (segment (start 54.530625 87.709375) (end 48.26 93.98) (width 0.4064) (layer B.Cu) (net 9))
 (segment (start 63.5 87.709375) (end 54.530625 87.709375) (width 0.4064) (layer B.Cu) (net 9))
 (segment (start 66.04 93.6625) (end 236.22 93.6625) (width 0.6096) (layer B.Cu) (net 8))
 (segment (start 66.04 93.6625) (end 65.484375 93.6625) (width 0.4064) (layer B.Cu) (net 8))
 (segment (start 65.484375 93.6625) (end 63.5 91.678125) (width 0.4064) (layer B.Cu) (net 8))
 (segment (start 53.101875 91.678125) (end 48.26 96.52) (width 0.4064) (layer B.Cu) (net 8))
 (segment (start 63.5 91.678125) (end 53.101875 91.678125) (width 0.4064) (layer B.Cu) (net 8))
 (segment (start 66.04 97.63125) (end 236.22 97.63125) (width 0.6096) (layer B.Cu) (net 7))
 (segment (start 66.04 97.63125) (end 65.484375 97.63125) (width 0.4064) (layer B.Cu) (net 7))
 (segment (start 65.484375 97.63125) (end 63.5 95.646875) (width 0.4064) (layer B.Cu) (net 7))
 (segment (start 51.673125 95.646875) (end 48.26 99.06) (width 0.4064) (layer B.Cu) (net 7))
 (segment (start 63.5 95.646875) (end 51.673125 95.646875) (width 0.4064) (layer B.Cu) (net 7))
 (segment (start 66.04 101.6) (end 236.22 101.6) (width 0.6096) (layer B.Cu) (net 6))
 (segment (start 66.04 101.6) (end 65.484375 101.6) (width 0.4064) (layer B.Cu) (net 6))
 (segment (start 65.484375 101.6) (end 63.5 99.615625) (width 0.4064) (layer B.Cu) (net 6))
 (segment (start 50.244375 99.615625) (end 48.26 101.6) (width 0.4064) (layer B.Cu) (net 6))
 (segment (start 63.5 99.615625) (end 50.244375 99.615625) (width 0.4064) (layer B.Cu) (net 6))
 (segment (start 66.04 105.56875) (end 236.22 105.56875) (width 0.6096) (layer B.Cu) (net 5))
 (segment (start 66.04 105.56875) (end 65.484375 105.56875) (width 0.4064) (layer B.Cu) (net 5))
 (segment (start 65.484375 105.56875) (end 63.5 103.584375) (width 0.4064) (layer B.Cu) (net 5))
 (segment (start 48.815625 103.584375) (end 48.26 104.14) (width 0.4064) (layer B.Cu) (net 5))
 (segment (start 63.5 103.584375) (end 48.815625 103.584375) (width 0.4064) (layer B.Cu) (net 5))
 (segment (start 66.04 109.5375) (end 236.22 109.5375) (width 0.6096) (layer B.Cu) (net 4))
 (segment (start 49.133125 107.553125) (end 48.26 106.68) (width 0.4064) (layer B.Cu) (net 4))
 (segment (start 63.5 107.553125) (end 49.133125 107.553125) (width 0.4064) (layer B.Cu) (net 4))
 (segment (start 65.484375 109.5375) (end 63.5 107.553125) (width 0.4064) (layer B.Cu) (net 4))
 (segment (start 66.04 109.5375) (end 65.484375 109.5375) (width 0.4064) (layer B.Cu) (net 4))
 (segment (start 66.04 113.50625) (end 236.22 113.50625) (width 0.6096) (layer B.Cu) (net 3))
 (segment (start 50.561875 111.521875) (end 48.26 109.22) (width 0.4064) (layer B.Cu) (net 3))
 (segment (start 63.5 111.521875) (end 50.561875 111.521875) (width 0.4064) (layer B.Cu) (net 3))
 (segment (start 65.484375 113.50625) (end 63.5 111.521875) (width 0.4064) (layer B.Cu) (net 3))
 (segment (start 66.04 113.50625) (end 65.484375 113.50625) (width 0.4064) (layer B.Cu) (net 3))
 (segment (start 66.04 117.475) (end 236.22 117.475) (width 0.6096) (layer B.Cu) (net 2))
 (segment (start 51.990625 115.490625) (end 48.26 111.76) (width 0.4064) (layer B.Cu) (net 2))
 (segment (start 63.5 115.490625) (end 51.990625 115.490625) (width 0.4064) (layer B.Cu) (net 2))
 (segment (start 65.484375 117.475) (end 63.5 115.490625) (width 0.4064) (layer B.Cu) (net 2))
 (segment (start 66.04 117.475) (end 65.484375 117.475) (width 0.4064) (layer B.Cu) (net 2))
 (segment (start 66.04 121.44375) (end 236.22 121.44375) (width 0.6096) (layer B.Cu) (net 1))
 (segment (start 66.04 121.44375) (end 65.484375 121.44375) (width 0.4064) (layer B.Cu) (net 1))
 (segment (start 65.484375 121.44375) (end 63.5 119.459375) (width 0.4064) (layer B.Cu) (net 1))
 (segment (start 53.419375 119.459375) (end 48.26 114.3) (width 0.4064) (layer B.Cu) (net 1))
 (segment (start 63.5 119.459375) (end 53.419375 119.459375) (width 0.4064) (layer B.Cu) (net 1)))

